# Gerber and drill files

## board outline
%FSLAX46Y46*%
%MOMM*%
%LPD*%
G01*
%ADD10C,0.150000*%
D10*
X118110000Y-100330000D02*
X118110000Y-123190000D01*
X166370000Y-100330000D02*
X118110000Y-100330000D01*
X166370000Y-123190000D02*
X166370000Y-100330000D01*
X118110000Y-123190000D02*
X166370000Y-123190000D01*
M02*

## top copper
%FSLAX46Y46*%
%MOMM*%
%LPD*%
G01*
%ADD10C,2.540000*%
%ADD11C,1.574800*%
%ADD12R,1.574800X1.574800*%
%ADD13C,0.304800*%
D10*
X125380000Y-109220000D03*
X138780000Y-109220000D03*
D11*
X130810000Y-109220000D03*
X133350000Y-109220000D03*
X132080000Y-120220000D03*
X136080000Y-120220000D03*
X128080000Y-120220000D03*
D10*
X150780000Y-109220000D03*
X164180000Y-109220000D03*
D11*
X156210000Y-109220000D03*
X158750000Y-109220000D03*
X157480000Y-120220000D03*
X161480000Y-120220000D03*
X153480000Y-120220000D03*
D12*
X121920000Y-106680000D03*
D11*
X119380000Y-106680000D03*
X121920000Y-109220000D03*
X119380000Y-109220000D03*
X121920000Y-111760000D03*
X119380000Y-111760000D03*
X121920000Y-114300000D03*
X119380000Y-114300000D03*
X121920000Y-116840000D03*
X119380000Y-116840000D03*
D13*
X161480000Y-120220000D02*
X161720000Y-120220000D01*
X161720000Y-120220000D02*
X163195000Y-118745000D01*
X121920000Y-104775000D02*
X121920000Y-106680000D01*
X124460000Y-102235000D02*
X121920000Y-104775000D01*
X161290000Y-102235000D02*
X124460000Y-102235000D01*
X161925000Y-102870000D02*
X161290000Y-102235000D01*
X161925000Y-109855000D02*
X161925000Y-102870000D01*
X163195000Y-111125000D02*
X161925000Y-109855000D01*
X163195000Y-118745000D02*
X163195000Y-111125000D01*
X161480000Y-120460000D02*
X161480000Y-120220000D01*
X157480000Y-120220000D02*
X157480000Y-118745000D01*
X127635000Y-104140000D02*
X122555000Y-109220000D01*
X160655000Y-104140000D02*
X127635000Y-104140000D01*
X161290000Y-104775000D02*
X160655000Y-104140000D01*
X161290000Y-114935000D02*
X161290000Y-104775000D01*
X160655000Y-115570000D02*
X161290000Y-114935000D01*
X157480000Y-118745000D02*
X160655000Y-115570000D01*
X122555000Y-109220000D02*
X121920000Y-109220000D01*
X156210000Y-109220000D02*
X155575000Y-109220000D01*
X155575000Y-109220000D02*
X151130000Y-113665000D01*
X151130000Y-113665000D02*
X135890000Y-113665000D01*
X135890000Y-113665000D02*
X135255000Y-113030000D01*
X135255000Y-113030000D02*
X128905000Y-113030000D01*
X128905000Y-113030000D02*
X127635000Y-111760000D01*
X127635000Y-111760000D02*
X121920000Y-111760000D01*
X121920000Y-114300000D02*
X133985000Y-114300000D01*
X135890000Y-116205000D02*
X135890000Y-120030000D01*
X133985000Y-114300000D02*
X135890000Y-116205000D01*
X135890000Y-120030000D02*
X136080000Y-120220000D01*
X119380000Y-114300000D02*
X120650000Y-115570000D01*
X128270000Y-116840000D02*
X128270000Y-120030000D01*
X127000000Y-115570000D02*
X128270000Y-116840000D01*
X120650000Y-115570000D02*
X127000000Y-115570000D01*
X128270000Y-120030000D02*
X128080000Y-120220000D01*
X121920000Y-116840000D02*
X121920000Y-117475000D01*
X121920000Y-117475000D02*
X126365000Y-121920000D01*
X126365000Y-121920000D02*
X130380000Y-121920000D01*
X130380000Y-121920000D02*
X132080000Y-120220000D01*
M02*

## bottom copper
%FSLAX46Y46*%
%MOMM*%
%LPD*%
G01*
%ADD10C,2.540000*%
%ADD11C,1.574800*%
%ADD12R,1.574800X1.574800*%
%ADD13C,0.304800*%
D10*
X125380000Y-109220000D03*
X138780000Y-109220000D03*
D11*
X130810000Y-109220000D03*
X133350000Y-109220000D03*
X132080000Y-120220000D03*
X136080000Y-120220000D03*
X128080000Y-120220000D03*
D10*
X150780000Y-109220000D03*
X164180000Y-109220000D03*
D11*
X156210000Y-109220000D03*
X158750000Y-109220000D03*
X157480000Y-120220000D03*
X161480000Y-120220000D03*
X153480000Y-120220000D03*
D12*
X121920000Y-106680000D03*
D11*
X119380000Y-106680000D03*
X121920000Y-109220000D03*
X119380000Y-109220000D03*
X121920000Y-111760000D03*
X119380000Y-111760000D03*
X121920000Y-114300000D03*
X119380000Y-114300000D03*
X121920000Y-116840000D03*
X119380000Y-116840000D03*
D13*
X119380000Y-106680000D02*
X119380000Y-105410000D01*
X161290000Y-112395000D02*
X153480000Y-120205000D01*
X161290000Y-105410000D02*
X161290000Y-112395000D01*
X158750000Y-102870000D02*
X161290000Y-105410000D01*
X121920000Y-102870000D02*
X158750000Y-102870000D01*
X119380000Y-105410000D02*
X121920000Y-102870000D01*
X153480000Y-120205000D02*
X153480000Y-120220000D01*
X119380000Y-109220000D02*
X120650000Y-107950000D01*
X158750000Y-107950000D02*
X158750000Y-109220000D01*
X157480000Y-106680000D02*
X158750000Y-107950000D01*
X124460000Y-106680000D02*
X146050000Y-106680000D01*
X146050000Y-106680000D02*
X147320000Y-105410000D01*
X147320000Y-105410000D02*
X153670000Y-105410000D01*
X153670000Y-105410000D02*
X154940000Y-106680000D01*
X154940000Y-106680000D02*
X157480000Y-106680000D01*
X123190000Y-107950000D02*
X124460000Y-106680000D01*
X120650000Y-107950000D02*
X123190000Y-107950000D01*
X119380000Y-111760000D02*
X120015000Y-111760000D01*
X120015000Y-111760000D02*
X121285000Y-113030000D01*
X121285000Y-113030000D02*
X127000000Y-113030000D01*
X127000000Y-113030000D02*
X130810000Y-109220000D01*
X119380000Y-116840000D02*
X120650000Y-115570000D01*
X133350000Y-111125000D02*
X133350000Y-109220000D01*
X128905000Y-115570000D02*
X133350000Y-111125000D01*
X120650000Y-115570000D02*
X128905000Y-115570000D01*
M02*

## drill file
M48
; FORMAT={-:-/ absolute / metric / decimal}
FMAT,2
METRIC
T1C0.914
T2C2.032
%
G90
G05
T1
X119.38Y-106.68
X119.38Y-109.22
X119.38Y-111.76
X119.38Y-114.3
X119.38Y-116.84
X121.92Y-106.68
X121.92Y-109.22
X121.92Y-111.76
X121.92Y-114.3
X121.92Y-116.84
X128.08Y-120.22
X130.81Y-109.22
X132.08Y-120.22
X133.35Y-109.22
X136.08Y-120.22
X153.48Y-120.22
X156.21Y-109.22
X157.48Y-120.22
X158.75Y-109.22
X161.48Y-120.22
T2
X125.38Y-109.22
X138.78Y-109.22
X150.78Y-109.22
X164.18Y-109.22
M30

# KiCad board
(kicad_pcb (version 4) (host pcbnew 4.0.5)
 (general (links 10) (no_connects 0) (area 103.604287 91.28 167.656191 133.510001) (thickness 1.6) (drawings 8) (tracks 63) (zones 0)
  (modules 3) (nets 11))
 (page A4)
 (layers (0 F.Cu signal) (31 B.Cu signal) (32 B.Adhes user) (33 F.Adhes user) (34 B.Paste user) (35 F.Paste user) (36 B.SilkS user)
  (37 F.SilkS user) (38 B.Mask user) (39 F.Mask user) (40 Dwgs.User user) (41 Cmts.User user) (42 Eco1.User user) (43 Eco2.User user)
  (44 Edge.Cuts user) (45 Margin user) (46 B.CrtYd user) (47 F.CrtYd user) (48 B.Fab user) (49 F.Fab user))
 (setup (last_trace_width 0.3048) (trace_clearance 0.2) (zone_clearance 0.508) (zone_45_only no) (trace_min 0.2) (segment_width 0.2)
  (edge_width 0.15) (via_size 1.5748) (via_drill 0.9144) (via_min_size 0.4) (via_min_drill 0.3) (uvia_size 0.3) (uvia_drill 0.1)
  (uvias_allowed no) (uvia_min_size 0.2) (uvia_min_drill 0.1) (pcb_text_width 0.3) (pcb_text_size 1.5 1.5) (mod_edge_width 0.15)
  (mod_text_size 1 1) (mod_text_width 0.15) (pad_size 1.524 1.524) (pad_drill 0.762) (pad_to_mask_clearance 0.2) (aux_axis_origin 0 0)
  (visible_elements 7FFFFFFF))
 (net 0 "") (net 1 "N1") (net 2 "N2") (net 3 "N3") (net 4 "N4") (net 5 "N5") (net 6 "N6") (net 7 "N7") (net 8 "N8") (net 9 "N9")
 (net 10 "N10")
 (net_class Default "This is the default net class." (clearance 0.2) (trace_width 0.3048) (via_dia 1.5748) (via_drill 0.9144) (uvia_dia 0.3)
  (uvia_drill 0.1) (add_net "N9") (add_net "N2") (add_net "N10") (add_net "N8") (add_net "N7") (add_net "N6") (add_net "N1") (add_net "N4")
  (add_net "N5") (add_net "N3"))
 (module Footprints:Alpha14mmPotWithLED (layer F.Cu) (at 132.08 109.22)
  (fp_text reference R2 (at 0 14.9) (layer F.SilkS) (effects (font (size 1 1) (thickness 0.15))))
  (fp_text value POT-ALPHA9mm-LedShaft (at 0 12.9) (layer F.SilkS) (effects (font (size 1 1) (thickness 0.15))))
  (pad "" thru_hole circle (at -6.7 0) (size 2.54 2.54) (drill 2.032) (layers *.Cu *.Mask F.SilkS))
  (pad "" thru_hole circle (at 6.7 0) (size 2.54 2.54) (drill 2.032) (layers *.Cu *.Mask F.SilkS))
  (pad 4 thru_hole circle (at -1.27 0) (size 1.5748 1.5748) (drill 0.9144) (layers *.Cu *.Mask F.SilkS) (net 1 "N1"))
  (pad 5 thru_hole circle (at 1.27 0) (size 1.5748 1.5748) (drill 0.9144) (layers *.Cu *.Mask F.SilkS) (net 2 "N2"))
  (pad 2 thru_hole circle (at 0 11) (size 1.5748 1.5748) (drill 0.9144) (layers *.Cu *.Mask F.SilkS) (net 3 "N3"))
  (pad 3 thru_hole circle (at 4 11) (size 1.5748 1.5748) (drill 0.9144) (layers *.Cu *.Mask F.SilkS) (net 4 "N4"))
  (pad 1 thru_hole circle (at -4 11) (size 1.5748 1.5748) (drill 0.9144) (layers *.Cu *.Mask F.SilkS) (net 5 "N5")))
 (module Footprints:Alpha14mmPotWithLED (layer F.Cu) (at 157.48 109.22)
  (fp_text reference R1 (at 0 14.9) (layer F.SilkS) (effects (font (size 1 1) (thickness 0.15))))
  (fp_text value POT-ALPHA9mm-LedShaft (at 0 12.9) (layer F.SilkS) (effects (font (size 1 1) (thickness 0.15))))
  (pad "" thru_hole circle (at -6.7 0) (size 2.54 2.54) (drill 2.032) (layers *.Cu *.Mask F.SilkS))
  (pad "" thru_hole circle (at 6.7 0) (size 2.54 2.54) (drill 2.032) (layers *.Cu *.Mask F.SilkS))
  (pad 4 thru_hole circle (at -1.27 0) (size 1.5748 1.5748) (drill 0.9144) (layers *.Cu *.Mask F.SilkS) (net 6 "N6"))
  (pad 5 thru_hole circle (at 1.27 0) (size 1.5748 1.5748) (drill 0.9144) (layers *.Cu *.Mask F.SilkS) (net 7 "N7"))
  (pad 2 thru_hole circle (at 0 11) (size 1.5748 1.5748) (drill 0.9144) (layers *.Cu *.Mask F.SilkS) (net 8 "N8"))
  (pad 3 thru_hole circle (at 4 11) (size 1.5748 1.5748) (drill 0.9144) (layers *.Cu *.Mask F.SilkS) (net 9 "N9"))
  (pad 1 thru_hole circle (at -4 11) (size 1.5748 1.5748) (drill 0.9144) (layers *.Cu *.Mask F.SilkS) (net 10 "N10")))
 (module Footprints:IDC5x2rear (layer F.Cu) (at 121.92 111.76 90)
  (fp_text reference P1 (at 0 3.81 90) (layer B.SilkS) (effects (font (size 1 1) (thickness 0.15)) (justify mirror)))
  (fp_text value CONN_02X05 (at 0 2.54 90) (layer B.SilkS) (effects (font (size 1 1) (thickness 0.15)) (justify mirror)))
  (pad 1 thru_hole rect (at 5.08 0 90) (size 1.5748 1.5748) (drill 0.9144) (layers *.Cu *.Mask B.SilkS) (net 9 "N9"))
  (pad 2 thru_hole circle (at 5.08 -2.54 90) (size 1.5748 1.5748) (drill 0.9144) (layers *.Cu *.Mask B.SilkS) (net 10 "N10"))
  (pad 3 thru_hole circle (at 2.54 0 90) (size 1.5748 1.5748) (drill 0.9144) (layers *.Cu *.Mask B.SilkS) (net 8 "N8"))
  (pad 4 thru_hole circle (at 2.54 -2.54 90) (size 1.5748 1.5748) (drill 0.9144) (layers *.Cu *.Mask B.SilkS) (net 7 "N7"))
  (pad 5 thru_hole circle (at 0 0 90) (size 1.5748 1.5748) (drill 0.9144) (layers *.Cu *.Mask B.SilkS) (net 6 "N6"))
  (pad 6 thru_hole circle (at 0 -2.54 90) (size 1.5748 1.5748) (drill 0.9144) (layers *.Cu *.Mask B.SilkS) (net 1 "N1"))
  (pad 7 thru_hole circle (at -2.54 0 90) (size 1.5748 1.5748) (drill 0.9144) (layers *.Cu *.Mask B.SilkS) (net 4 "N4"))
  (pad 8 thru_hole circle (at -2.54 -2.54 90) (size 1.5748 1.5748) (drill 0.9144) (layers *.Cu *.Mask B.SilkS) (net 5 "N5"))
  (pad 9 thru_hole circle (at -5.08 0 90) (size 1.5748 1.5748) (drill 0.9144) (layers *.Cu *.Mask B.SilkS) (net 3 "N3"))
  (pad 10 thru_hole circle (at -5.08 -2.54 90) (size 1.5748 1.5748) (drill 0.9144) (layers *.Cu *.Mask B.SilkS) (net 2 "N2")))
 (gr_line (start 118.11 100.33) (end 118.11 123.19) (angle 90) (layer Edge.Cuts) (width 0.15))
 (gr_line (start 166.37 100.33) (end 118.11 100.33) (angle 90) (layer Edge.Cuts) (width 0.15))
 (gr_line (start 166.37 123.19) (end 166.37 100.33) (angle 90) (layer Edge.Cuts) (width 0.15))
 (gr_line (start 118.11 123.19) (end 166.37 123.19) (angle 90) (layer Edge.Cuts) (width 0.15))
 (segment (start 161.48 120.22) (end 161.72 120.22) (width 0.3048) (layer F.Cu) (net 9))
 (segment (start 161.72 120.22) (end 163.195 118.745) (width 0.3048) (layer F.Cu) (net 9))
 (segment (start 121.92 104.775) (end 121.92 106.68) (width 0.3048) (layer F.Cu) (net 9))
 (segment (start 124.46 102.235) (end 121.92 104.775) (width 0.3048) (layer F.Cu) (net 9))
 (segment (start 161.29 102.235) (end 124.46 102.235) (width 0.3048) (layer F.Cu) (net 9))
 (segment (start 161.925 102.87) (end 161.29 102.235) (width 0.3048) (layer F.Cu) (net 9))
 (segment (start 161.925 109.855) (end 161.925 102.87) (width 0.3048) (layer F.Cu) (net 9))
 (segment (start 163.195 111.125) (end 161.925 109.855) (width 0.3048) (layer F.Cu) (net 9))
 (segment (start 163.195 118.745) (end 163.195 111.125) (width 0.3048) (layer F.Cu) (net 9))
 (segment (start 161.48 120.46) (end 161.48 120.22) (width 0.3048) (layer F.Cu) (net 9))
 (segment (start 119.38 106.68) (end 119.38 105.41) (width 0.3048) (layer B.Cu) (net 10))
 (segment (start 161.29 112.395) (end 153.48 120.205) (width 0.3048) (layer B.Cu) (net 10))
 (segment (start 161.29 105.41) (end 161.29 112.395) (width 0.3048) (layer B.Cu) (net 10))
 (segment (start 158.75 102.87) (end 161.29 105.41) (width 0.3048) (layer B.Cu) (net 10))
 (segment (start 121.92 102.87) (end 158.75 102.87) (width 0.3048) (layer B.Cu) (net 10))
 (segment (start 119.38 105.41) (end 121.92 102.87) (width 0.3048) (layer B.Cu) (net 10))
 (segment (start 153.48 120.205) (end 153.48 120.22) (width 0.3048) (layer B.Cu) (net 10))
 (segment (start 157.48 120.22) (end 157.48 118.745) (width 0.3048) (layer F.Cu) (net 8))
 (segment (start 127.635 104.14) (end 122.555 109.22) (width 0.3048) (layer F.Cu) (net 8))
 (segment (start 160.655 104.14) (end 127.635 104.14) (width 0.3048) (layer F.Cu) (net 8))
 (segment (start 161.29 104.775) (end 160.655 104.14) (width 0.3048) (layer F.Cu) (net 8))
 (segment (start 161.29 114.935) (end 161.29 104.775) (width 0.3048) (layer F.Cu) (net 8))
 (segment (start 160.655 115.57) (end 161.29 114.935) (width 0.3048) (layer F.Cu) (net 8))
 (segment (start 157.48 118.745) (end 160.655 115.57) (width 0.3048) (layer F.Cu) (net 8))
 (segment (start 122.555 109.22) (end 121.92 109.22) (width 0.3048) (layer F.Cu) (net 8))
 (segment (start 119.38 109.22) (end 120.65 107.95) (width 0.3048) (layer B.Cu) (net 7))
 (segment (start 158.75 107.95) (end 158.75 109.22) (width 0.3048) (layer B.Cu) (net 7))
 (segment (start 157.48 106.68) (end 158.75 107.95) (width 0.3048) (layer B.Cu) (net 7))
 (segment (start 124.46 106.68) (end 146.05 106.68) (width 0.3048) (layer B.Cu) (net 7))
 (segment (start 146.05 106.68) (end 147.32 105.41) (width 0.3048) (layer B.Cu) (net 7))
 (segment (start 147.32 105.41) (end 153.67 105.41) (width 0.3048) (layer B.Cu) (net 7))
 (segment (start 153.67 105.41) (end 154.94 106.68) (width 0.3048) (layer B.Cu) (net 7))
 (segment (start 154.94 106.68) (end 157.48 106.68) (width 0.3048) (layer B.Cu) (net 7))
 (segment (start 123.19 107.95) (end 124.46 106.68) (width 0.3048) (layer B.Cu) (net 7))
 (segment (start 120.65 107.95) (end 123.19 107.95) (width 0.3048) (layer B.Cu) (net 7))
 (segment (start 156.21 109.22) (end 155.575 109.22) (width 0.3048) (layer F.Cu) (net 6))
 (segment (start 155.575 109.22) (end 151.13 113.665) (width 0.3048) (layer F.Cu) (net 6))
 (segment (start 151.13 113.665) (end 135.89 113.665) (width 0.3048) (layer F.Cu) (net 6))
 (segment (start 135.89 113.665) (end 135.255 113.03) (width 0.3048) (layer F.Cu) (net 6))
 (segment (start 135.255 113.03) (end 128.905 113.03) (width 0.3048) (layer F.Cu) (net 6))
 (segment (start 128.905 113.03) (end 127.635 111.76) (width 0.3048) (layer F.Cu) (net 6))
 (segment (start 127.635 111.76) (end 121.92 111.76) (width 0.3048) (layer F.Cu) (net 6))
 (segment (start 119.38 111.76) (end 120.015 111.76) (width 0.3048) (layer B.Cu) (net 1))
 (segment (start 120.015 111.76) (end 121.285 113.03) (width 0.3048) (layer B.Cu) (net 1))
 (segment (start 121.285 113.03) (end 127 113.03) (width 0.3048) (layer B.Cu) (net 1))
 (segment (start 127 113.03) (end 130.81 109.22) (width 0.3048) (layer B.Cu) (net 1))
 (segment (start 121.92 114.3) (end 133.985 114.3) (width 0.3048) (layer F.Cu) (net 4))
 (segment (start 135.89 116.205) (end 135.89 120.03) (width 0.3048) (layer F.Cu) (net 4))
 (segment (start 133.985 114.3) (end 135.89 116.205) (width 0.3048) (layer F.Cu) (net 4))
 (segment (start 135.89 120.03) (end 136.08 120.22) (width 0.3048) (layer F.Cu) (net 4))
 (segment (start 119.38 114.3) (end 120.65 115.57) (width 0.3048) (layer F.Cu) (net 5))
 (segment (start 128.27 116.84) (end 128.27 120.03) (width 0.3048) (layer F.Cu) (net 5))
 (segment (start 127 115.57) (end 128.27 116.84) (width 0.3048) (layer F.Cu) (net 5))
 (segment (start 120.65 115.57) (end 127 115.57) (width 0.3048) (layer F.Cu) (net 5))
 (segment (start 128.27 120.03) (end 128.08 120.22) (width 0.3048) (layer F.Cu) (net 5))
 (segment (start 121.92 116.84) (end 121.92 117.475) (width 0.3048) (layer F.Cu) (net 3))
 (segment (start 121.92 117.475) (end 126.365 121.92) (width 0.3048) (layer F.Cu) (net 3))
 (segment (start 126.365 121.92) (end 130.38 121.92) (width 0.3048) (layer F.Cu) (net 3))
 (segment (start 130.38 121.92) (end 132.08 120.22) (width 0.3048) (layer F.Cu) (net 3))
 (segment (start 119.38 116.84) (end 120.65 115.57) (width 0.3048) (layer B.Cu) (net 2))
 (segment (start 133.35 111.125) (end 133.35 109.22) (width 0.3048) (layer B.Cu) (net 2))
 (segment (start 128.905 115.57) (end 133.35 111.125) (width 0.3048) (layer B.Cu) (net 2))
 (segment (start 120.65 115.57) (end 128.905 115.57) (width 0.3048) (layer B.Cu) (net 2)))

